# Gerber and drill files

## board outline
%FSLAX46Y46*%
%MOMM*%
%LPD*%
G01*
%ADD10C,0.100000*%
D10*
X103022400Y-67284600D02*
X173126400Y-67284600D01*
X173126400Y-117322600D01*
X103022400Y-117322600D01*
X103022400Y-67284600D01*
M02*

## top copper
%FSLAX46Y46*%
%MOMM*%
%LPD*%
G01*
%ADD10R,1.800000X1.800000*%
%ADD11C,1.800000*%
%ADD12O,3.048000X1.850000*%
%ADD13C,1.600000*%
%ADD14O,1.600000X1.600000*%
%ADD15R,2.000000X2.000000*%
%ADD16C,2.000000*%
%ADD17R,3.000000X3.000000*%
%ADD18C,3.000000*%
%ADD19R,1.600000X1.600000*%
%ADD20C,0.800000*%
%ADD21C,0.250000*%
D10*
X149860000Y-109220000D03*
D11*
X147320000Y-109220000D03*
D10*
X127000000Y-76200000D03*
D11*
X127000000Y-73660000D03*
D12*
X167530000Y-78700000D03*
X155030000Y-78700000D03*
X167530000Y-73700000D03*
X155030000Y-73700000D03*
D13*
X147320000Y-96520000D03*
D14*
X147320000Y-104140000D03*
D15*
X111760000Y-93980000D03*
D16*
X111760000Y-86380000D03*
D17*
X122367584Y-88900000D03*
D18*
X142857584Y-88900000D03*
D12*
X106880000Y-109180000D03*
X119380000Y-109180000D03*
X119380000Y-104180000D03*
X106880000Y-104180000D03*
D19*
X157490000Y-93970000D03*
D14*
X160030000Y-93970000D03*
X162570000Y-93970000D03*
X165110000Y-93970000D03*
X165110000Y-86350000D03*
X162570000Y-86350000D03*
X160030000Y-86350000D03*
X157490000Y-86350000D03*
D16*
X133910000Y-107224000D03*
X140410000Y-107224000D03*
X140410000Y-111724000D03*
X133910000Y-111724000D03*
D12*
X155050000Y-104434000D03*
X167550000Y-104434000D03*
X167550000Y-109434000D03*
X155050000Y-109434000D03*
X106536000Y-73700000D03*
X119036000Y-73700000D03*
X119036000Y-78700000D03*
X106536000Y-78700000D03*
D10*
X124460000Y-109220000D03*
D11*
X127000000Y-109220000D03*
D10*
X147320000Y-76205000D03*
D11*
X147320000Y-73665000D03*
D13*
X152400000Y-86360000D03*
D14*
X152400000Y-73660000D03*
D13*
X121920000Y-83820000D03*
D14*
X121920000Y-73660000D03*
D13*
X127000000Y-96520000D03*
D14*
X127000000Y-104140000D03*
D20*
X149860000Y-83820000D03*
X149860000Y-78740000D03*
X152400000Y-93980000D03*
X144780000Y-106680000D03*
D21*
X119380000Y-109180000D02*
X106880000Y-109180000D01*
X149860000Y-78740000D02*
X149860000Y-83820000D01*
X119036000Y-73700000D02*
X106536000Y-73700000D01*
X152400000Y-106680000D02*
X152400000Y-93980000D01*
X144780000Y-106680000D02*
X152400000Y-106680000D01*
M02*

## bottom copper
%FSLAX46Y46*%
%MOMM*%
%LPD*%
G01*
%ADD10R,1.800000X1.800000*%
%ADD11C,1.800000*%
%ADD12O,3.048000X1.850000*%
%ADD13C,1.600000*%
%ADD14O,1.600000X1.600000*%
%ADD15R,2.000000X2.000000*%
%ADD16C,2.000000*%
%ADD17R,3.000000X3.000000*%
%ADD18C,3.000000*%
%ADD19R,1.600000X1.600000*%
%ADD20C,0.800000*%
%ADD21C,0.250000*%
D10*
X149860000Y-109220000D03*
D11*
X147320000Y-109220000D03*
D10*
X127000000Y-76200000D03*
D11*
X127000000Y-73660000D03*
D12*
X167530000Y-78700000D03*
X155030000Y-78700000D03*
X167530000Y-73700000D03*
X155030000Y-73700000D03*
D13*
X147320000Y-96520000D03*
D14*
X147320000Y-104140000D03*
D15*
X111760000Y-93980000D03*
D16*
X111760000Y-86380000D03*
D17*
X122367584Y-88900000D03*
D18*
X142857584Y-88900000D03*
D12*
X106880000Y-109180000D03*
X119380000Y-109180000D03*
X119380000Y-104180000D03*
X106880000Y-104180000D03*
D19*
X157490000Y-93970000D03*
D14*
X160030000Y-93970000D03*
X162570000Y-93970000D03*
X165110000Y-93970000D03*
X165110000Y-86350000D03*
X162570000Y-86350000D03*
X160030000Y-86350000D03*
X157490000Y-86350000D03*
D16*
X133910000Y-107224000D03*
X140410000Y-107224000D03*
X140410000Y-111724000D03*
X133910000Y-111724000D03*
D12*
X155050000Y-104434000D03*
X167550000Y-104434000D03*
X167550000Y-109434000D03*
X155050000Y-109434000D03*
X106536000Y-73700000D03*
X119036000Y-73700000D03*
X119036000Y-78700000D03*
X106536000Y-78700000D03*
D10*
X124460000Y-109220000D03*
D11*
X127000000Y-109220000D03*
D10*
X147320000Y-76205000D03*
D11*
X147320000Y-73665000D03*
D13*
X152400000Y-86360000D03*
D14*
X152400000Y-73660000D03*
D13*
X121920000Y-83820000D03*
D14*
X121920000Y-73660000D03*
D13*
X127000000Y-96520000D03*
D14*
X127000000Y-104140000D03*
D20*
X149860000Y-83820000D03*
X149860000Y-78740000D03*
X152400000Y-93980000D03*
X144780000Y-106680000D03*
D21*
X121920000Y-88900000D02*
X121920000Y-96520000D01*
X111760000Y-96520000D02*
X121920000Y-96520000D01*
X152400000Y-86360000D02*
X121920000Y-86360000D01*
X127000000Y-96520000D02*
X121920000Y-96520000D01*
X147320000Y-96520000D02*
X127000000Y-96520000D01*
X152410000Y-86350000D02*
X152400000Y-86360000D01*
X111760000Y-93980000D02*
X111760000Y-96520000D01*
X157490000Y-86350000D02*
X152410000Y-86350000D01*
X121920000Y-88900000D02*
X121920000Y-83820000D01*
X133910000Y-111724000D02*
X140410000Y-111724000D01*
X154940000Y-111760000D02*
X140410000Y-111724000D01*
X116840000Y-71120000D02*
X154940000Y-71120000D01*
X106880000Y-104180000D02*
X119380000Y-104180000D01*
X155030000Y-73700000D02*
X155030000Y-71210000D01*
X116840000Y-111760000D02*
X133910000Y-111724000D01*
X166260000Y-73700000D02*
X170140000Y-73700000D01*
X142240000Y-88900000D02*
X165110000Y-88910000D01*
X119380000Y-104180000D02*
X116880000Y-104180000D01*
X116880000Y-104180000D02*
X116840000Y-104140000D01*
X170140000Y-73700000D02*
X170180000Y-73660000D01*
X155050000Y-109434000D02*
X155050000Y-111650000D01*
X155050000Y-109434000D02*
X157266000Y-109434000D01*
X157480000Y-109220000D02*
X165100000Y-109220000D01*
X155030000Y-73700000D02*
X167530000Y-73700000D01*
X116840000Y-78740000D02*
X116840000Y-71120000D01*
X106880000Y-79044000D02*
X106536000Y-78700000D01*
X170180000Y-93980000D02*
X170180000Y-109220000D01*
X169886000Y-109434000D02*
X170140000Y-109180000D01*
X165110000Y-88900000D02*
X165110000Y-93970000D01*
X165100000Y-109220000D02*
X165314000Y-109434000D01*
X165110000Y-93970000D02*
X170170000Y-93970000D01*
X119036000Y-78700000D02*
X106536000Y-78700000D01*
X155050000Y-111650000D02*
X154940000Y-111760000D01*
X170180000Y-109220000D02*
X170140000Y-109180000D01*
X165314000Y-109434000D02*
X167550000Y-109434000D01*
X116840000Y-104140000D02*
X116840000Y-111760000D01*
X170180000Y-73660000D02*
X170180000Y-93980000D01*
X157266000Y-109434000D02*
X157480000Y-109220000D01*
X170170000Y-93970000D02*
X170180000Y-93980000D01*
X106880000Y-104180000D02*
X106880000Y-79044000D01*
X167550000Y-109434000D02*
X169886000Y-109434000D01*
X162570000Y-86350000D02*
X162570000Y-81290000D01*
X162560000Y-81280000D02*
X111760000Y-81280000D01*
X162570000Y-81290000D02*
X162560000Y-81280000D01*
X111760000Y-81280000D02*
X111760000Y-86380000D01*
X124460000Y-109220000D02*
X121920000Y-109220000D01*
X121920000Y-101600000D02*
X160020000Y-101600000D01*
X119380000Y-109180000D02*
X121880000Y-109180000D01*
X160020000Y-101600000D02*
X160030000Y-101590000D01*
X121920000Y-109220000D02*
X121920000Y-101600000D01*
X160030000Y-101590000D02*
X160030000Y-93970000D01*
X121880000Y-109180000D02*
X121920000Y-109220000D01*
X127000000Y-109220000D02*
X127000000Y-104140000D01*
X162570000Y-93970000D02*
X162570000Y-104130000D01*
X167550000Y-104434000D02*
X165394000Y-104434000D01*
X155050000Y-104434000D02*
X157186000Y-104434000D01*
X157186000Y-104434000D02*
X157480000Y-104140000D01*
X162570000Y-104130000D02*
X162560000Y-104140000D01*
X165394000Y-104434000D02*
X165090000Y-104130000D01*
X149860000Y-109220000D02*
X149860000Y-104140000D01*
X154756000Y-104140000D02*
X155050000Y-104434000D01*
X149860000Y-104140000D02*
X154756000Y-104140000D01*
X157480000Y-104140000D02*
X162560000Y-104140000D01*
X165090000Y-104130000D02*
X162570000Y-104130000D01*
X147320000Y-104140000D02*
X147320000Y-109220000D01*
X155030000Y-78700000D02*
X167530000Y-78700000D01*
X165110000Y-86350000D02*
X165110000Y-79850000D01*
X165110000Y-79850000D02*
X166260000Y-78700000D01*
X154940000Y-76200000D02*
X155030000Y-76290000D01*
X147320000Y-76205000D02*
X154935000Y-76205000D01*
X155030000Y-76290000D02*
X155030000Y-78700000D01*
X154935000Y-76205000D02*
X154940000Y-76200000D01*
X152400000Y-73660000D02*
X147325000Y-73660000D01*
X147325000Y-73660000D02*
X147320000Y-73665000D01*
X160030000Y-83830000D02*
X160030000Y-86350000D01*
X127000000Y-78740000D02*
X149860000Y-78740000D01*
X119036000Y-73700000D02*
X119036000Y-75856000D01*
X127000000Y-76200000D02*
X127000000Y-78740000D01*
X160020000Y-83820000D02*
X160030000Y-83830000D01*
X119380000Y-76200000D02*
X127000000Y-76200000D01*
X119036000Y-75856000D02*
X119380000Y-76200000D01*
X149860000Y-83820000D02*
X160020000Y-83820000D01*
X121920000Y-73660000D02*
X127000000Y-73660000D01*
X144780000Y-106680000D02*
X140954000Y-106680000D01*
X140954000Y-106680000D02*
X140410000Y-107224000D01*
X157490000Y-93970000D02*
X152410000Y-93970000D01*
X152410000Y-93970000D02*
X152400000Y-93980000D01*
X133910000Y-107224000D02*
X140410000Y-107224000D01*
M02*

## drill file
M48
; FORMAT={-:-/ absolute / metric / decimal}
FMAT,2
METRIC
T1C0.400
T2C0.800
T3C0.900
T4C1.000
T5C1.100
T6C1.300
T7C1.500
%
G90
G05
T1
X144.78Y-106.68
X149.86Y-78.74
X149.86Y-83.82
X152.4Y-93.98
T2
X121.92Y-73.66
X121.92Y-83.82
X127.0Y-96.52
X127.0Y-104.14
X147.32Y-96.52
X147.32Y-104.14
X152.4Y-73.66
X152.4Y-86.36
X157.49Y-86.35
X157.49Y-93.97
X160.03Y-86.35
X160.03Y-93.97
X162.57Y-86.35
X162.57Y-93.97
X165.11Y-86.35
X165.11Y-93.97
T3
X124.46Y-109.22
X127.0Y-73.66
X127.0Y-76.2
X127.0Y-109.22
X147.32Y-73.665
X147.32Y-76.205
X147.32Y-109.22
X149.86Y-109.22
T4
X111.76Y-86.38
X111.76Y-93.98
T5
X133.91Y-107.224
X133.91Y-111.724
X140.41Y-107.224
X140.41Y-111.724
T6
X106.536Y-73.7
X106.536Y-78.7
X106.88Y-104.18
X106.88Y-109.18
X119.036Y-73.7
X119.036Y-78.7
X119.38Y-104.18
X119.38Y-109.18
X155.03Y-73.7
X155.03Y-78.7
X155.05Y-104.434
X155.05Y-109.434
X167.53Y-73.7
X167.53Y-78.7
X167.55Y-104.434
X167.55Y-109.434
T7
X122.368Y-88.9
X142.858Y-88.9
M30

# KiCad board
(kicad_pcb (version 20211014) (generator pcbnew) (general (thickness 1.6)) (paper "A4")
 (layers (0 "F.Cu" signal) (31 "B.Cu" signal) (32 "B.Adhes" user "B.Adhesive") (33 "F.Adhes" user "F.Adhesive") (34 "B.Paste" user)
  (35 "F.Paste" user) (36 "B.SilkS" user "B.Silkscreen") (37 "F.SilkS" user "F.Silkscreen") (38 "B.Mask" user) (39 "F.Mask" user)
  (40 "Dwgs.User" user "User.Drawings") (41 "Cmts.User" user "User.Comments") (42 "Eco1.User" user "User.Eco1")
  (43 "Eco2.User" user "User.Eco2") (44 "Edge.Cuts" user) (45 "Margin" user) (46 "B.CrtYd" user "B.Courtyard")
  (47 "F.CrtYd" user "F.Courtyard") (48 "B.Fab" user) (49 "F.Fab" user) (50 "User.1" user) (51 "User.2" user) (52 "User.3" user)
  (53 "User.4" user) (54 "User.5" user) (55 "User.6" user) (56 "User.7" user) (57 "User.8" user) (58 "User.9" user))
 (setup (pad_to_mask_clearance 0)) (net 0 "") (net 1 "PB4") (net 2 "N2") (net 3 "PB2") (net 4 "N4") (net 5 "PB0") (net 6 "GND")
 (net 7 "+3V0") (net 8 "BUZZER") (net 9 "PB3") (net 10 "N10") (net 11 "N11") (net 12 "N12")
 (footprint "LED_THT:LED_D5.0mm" (layer "F.Cu") (at 149.86 109.22 180)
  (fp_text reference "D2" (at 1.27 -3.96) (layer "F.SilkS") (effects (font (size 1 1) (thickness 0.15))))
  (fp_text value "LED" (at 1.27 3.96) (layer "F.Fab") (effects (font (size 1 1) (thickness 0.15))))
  (pad "1" thru_hole rect (at 0 0 180) (size 1.8 1.8) (drill 0.9) (layers *.Cu *.Mask) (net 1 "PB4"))
  (pad "2" thru_hole circle (at 2.54 0 180) (size 1.8 1.8) (drill 0.9) (layers *.Cu *.Mask) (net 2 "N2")))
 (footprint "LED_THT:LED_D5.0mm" (layer "F.Cu") (at 127 76.2 90)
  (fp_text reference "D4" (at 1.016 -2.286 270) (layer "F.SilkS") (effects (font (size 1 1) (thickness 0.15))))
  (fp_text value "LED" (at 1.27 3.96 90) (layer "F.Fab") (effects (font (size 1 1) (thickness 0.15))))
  (pad "1" thru_hole rect (at 0 0 90) (size 1.8 1.8) (drill 0.9) (layers *.Cu *.Mask) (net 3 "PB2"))
  (pad "2" thru_hole circle (at 2.54 0 90) (size 1.8 1.8) (drill 0.9) (layers *.Cu *.Mask) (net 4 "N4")))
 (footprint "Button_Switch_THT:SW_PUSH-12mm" (layer "F.Cu") (at 167.53 78.7 180)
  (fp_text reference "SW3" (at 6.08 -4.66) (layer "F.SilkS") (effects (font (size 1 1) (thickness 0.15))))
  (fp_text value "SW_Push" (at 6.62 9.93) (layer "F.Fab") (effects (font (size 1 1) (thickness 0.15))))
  (pad "1" thru_hole oval (at 0 0 180) (size 3.048 1.85) (drill 1.3) (layers *.Cu *.Mask) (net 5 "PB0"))
  (pad "1" thru_hole oval (at 12.5 0 180) (size 3.048 1.85) (drill 1.3) (layers *.Cu *.Mask) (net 5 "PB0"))
  (pad "2" thru_hole oval (at 0 5 180) (size 3.048 1.85) (drill 1.3) (layers *.Cu *.Mask) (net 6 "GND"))
  (pad "2" thru_hole oval (at 12.5 5 180) (size 3.048 1.85) (drill 1.3) (layers *.Cu *.Mask) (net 6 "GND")))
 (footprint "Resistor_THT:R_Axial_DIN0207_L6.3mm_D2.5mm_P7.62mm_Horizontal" (layer "F.Cu") (at 147.32 96.52 -90)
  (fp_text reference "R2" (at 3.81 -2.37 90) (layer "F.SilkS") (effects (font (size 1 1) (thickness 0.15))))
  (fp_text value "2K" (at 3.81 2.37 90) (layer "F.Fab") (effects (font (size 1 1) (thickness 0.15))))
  (pad "1" thru_hole circle (at 0 0 270) (size 1.6 1.6) (drill 0.8) (layers *.Cu *.Mask) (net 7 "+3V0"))
  (pad "2" thru_hole oval (at 7.62 0 270) (size 1.6 1.6) (drill 0.8) (layers *.Cu *.Mask) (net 2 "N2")))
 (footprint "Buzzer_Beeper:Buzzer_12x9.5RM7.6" (layer "F.Cu") (at 111.76 93.98 90)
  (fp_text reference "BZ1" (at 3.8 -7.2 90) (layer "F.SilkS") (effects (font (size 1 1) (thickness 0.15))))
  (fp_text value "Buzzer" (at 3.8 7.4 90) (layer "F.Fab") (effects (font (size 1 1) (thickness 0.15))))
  (pad "1" thru_hole rect (at 0 0 90) (size 2 2) (drill 1) (layers *.Cu *.Mask) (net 7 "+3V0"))
  (pad "2" thru_hole circle (at 7.6 0 90) (size 2 2) (drill 1) (layers *.Cu *.Mask) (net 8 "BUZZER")))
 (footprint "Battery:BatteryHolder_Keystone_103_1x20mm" (layer "F.Cu") (at 122.367584 88.9)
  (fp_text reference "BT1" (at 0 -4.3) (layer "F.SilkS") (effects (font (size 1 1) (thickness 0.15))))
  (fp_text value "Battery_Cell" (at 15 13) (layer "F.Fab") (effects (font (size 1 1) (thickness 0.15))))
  (pad "1" thru_hole rect (at 0 0) (size 3 3) (drill 1.5) (layers *.Cu *.Mask) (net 7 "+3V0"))
  (pad "2" thru_hole circle (at 20.49 0) (size 3 3) (drill 1.5) (layers *.Cu *.Mask) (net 6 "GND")))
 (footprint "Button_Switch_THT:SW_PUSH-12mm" (layer "F.Cu") (at 119.38 109.18 180)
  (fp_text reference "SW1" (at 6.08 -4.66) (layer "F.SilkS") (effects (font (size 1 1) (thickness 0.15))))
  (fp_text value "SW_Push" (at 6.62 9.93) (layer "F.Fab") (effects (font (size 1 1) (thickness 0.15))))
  (pad "1" thru_hole oval (at 12.5 0 180) (size 3.048 1.85) (drill 1.3) (layers *.Cu *.Mask) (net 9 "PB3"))
  (pad "1" thru_hole oval (at 0 0 180) (size 3.048 1.85) (drill 1.3) (layers *.Cu *.Mask) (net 9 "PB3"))
  (pad "2" thru_hole oval (at 0 5 180) (size 3.048 1.85) (drill 1.3) (layers *.Cu *.Mask) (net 6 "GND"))
  (pad "2" thru_hole oval (at 12.5 5 180) (size 3.048 1.85) (drill 1.3) (layers *.Cu *.Mask) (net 6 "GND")))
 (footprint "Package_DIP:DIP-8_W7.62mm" (layer "F.Cu") (at 157.49 93.97 90)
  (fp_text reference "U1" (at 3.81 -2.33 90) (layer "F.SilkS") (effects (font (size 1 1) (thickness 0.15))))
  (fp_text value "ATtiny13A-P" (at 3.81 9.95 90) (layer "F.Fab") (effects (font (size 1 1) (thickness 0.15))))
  (pad "1" thru_hole rect (at 0 0 90) (size 1.6 1.6) (drill 0.8) (layers *.Cu *.Mask) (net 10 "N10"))
  (pad "2" thru_hole oval (at 0 2.54 90) (size 1.6 1.6) (drill 0.8) (layers *.Cu *.Mask) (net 9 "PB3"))
  (pad "3" thru_hole oval (at 0 5.08 90) (size 1.6 1.6) (drill 0.8) (layers *.Cu *.Mask) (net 1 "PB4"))
  (pad "4" thru_hole oval (at 0 7.62 90) (size 1.6 1.6) (drill 0.8) (layers *.Cu *.Mask) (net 6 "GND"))
  (pad "5" thru_hole oval (at 7.62 7.62 90) (size 1.6 1.6) (drill 0.8) (layers *.Cu *.Mask) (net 5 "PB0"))
  (pad "6" thru_hole oval (at 7.62 5.08 90) (size 1.6 1.6) (drill 0.8) (layers *.Cu *.Mask) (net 8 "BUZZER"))
  (pad "7" thru_hole oval (at 7.62 2.54 90) (size 1.6 1.6) (drill 0.8) (layers *.Cu *.Mask) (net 3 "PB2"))
  (pad "8" thru_hole oval (at 7.62 0 90) (size 1.6 1.6) (drill 0.8) (layers *.Cu *.Mask) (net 7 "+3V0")))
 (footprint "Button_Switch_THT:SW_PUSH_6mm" (layer "F.Cu") (at 133.91 107.224)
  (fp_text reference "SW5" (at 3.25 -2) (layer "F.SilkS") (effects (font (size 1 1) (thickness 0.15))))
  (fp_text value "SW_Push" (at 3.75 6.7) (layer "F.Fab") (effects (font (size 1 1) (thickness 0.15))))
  (pad "1" thru_hole circle (at 0 0 90) (size 2 2) (drill 1.1) (layers *.Cu *.Mask) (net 10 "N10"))
  (pad "1" thru_hole circle (at 6.5 0 90) (size 2 2) (drill 1.1) (layers *.Cu *.Mask) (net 10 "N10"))
  (pad "2" thru_hole circle (at 6.5 4.5 90) (size 2 2) (drill 1.1) (layers *.Cu *.Mask) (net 6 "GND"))
  (pad "2" thru_hole circle (at 0 4.5 90) (size 2 2) (drill 1.1) (layers *.Cu *.Mask) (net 6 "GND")))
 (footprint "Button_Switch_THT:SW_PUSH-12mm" (layer "F.Cu") (at 155.05 104.434)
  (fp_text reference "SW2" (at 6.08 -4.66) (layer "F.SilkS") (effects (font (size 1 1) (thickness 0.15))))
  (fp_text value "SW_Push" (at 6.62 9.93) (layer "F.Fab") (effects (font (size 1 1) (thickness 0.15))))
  (pad "1" thru_hole oval (at 0 0) (size 3.048 1.85) (drill 1.3) (layers *.Cu *.Mask) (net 1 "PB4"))
  (pad "1" thru_hole oval (at 12.5 0) (size 3.048 1.85) (drill 1.3) (layers *.Cu *.Mask) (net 1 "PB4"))
  (pad "2" thru_hole oval (at 12.5 5) (size 3.048 1.85) (drill 1.3) (layers *.Cu *.Mask) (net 6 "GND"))
  (pad "2" thru_hole oval (at 0 5) (size 3.048 1.85) (drill 1.3) (layers *.Cu *.Mask) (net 6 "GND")))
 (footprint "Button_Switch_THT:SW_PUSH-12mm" (layer "F.Cu") (at 106.536 73.7)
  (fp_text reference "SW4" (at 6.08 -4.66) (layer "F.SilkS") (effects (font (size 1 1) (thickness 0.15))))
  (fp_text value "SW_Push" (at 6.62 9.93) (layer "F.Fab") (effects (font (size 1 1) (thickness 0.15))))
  (pad "1" thru_hole oval (at 0 0) (size 3.048 1.85) (drill 1.3) (layers *.Cu *.Mask) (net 3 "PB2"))
  (pad "1" thru_hole oval (at 12.5 0) (size 3.048 1.85) (drill 1.3) (layers *.Cu *.Mask) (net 3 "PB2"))
  (pad "2" thru_hole oval (at 12.5 5) (size 3.048 1.85) (drill 1.3) (layers *.Cu *.Mask) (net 6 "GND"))
  (pad "2" thru_hole oval (at 0 5) (size 3.048 1.85) (drill 1.3) (layers *.Cu *.Mask) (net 6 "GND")))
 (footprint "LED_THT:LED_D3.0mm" (layer "F.Cu") (at 124.46 109.22)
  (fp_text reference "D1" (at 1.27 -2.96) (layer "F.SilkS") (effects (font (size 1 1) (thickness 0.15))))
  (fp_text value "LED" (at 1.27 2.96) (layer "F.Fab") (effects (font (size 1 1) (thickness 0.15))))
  (pad "1" thru_hole rect (at 0 0) (size 1.8 1.8) (drill 0.9) (layers *.Cu *.Mask) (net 9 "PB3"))
  (pad "2" thru_hole circle (at 2.54 0) (size 1.8 1.8) (drill 0.9) (layers *.Cu *.Mask) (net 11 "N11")))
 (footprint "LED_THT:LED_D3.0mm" (layer "F.Cu") (at 147.32 76.205 90)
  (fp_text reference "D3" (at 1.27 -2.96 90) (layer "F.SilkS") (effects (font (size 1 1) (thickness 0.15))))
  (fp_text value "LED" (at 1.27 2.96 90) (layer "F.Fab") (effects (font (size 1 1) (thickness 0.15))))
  (pad "1" thru_hole rect (at 0 0 90) (size 1.8 1.8) (drill 0.9) (layers *.Cu *.Mask) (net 5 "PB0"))
  (pad "2" thru_hole circle (at 2.54 0 90) (size 1.8 1.8) (drill 0.9) (layers *.Cu *.Mask) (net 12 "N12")))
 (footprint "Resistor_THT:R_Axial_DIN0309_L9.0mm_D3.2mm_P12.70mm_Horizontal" (layer "F.Cu") (at 152.4 86.36 90)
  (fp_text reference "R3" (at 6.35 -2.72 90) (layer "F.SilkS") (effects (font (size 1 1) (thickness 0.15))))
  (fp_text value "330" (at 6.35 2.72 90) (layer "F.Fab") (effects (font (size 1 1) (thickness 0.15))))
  (pad "1" thru_hole circle (at 0 0 90) (size 1.6 1.6) (drill 0.8) (layers *.Cu *.Mask) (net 7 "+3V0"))
  (pad "2" thru_hole oval (at 12.7 0 90) (size 1.6 1.6) (drill 0.8) (layers *.Cu *.Mask) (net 12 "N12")))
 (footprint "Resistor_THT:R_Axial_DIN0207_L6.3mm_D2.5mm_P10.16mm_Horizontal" (layer "F.Cu") (at 121.92 83.82 90)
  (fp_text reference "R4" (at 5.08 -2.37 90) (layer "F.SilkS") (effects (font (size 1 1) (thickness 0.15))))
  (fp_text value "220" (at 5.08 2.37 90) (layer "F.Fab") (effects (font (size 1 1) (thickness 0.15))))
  (pad "1" thru_hole circle (at 0 0 90) (size 1.6 1.6) (drill 0.8) (layers *.Cu *.Mask) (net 7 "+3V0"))
  (pad "2" thru_hole oval (at 10.16 0 90) (size 1.6 1.6) (drill 0.8) (layers *.Cu *.Mask) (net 4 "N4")))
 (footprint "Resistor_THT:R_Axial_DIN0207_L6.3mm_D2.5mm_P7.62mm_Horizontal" (layer "F.Cu") (at 127 96.52 -90)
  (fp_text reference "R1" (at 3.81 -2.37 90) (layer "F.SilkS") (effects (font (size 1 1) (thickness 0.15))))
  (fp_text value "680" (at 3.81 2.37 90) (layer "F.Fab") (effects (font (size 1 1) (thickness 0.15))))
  (pad "1" thru_hole circle (at 0 0 270) (size 1.6 1.6) (drill 0.8) (layers *.Cu *.Mask) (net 7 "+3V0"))
  (pad "2" thru_hole oval (at 7.62 0 270) (size 1.6 1.6) (drill 0.8) (layers *.Cu *.Mask) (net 11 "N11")))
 (gr_rect (start 103.0224 67.2846) (end 173.1264 117.3226) (layer "Edge.Cuts") (width 0.1) (fill none))
 (segment (start 121.92 88.9) (end 121.92 96.52) (width 0.25) (layer "B.Cu") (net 7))
 (segment (start 111.76 96.52) (end 121.92 96.52) (width 0.25) (layer "B.Cu") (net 7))
 (segment (start 152.4 86.36) (end 121.92 86.36) (width 0.25) (layer "B.Cu") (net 7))
 (segment (start 127 96.52) (end 121.92 96.52) (width 0.25) (layer "B.Cu") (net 7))
 (segment (start 147.32 96.52) (end 127 96.52) (width 0.25) (layer "B.Cu") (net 7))
 (segment (start 152.41 86.35) (end 152.4 86.36) (width 0.25) (layer "B.Cu") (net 7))
 (segment (start 111.76 93.98) (end 111.76 96.52) (width 0.25) (layer "B.Cu") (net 7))
 (segment (start 157.49 86.35) (end 152.41 86.35) (width 0.25) (layer "B.Cu") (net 7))
 (segment (start 121.92 88.9) (end 121.92 83.82) (width 0.25) (layer "B.Cu") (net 7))
 (segment (start 133.91 111.724) (end 140.41 111.724) (width 0.25) (layer "B.Cu") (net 6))
 (segment (start 154.94 111.76) (end 140.41 111.724) (width 0.25) (layer "B.Cu") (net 6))
 (segment (start 116.84 71.12) (end 154.94 71.12) (width 0.25) (layer "B.Cu") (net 6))
 (segment (start 106.88 104.18) (end 119.38 104.18) (width 0.25) (layer "B.Cu") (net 6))
 (segment (start 155.03 73.7) (end 155.03 71.21) (width 0.25) (layer "B.Cu") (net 6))
 (segment (start 116.84 111.76) (end 133.91 111.724) (width 0.25) (layer "B.Cu") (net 6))
 (segment (start 166.26 73.7) (end 170.14 73.7) (width 0.25) (layer "B.Cu") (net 6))
 (segment (start 142.24 88.9) (end 165.11 88.91) (width 0.25) (layer "B.Cu") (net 6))
 (segment (start 119.38 104.18) (end 116.88 104.18) (width 0.25) (layer "B.Cu") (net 6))
 (segment (start 116.88 104.18) (end 116.84 104.14) (width 0.25) (layer "B.Cu") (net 6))
 (segment (start 170.14 73.7) (end 170.18 73.66) (width 0.25) (layer "B.Cu") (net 6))
 (segment (start 155.05 109.434) (end 155.05 111.65) (width 0.25) (layer "B.Cu") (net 6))
 (segment (start 155.05 109.434) (end 157.266 109.434) (width 0.25) (layer "B.Cu") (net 6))
 (segment (start 157.48 109.22) (end 165.1 109.22) (width 0.25) (layer "B.Cu") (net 6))
 (segment (start 155.03 73.7) (end 167.53 73.7) (width 0.25) (layer "B.Cu") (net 6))
 (segment (start 116.84 78.74) (end 116.84 71.12) (width 0.25) (layer "B.Cu") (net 6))
 (segment (start 106.88 79.044) (end 106.536 78.7) (width 0.25) (layer "B.Cu") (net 6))
 (segment (start 170.18 93.98) (end 170.18 109.22) (width 0.25) (layer "B.Cu") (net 6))
 (segment (start 169.886 109.434) (end 170.14 109.18) (width 0.25) (layer "B.Cu") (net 6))
 (segment (start 165.11 88.9) (end 165.11 93.97) (width 0.25) (layer "B.Cu") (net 6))
 (segment (start 165.1 109.22) (end 165.314 109.434) (width 0.25) (layer "B.Cu") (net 6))
 (segment (start 165.11 93.97) (end 170.17 93.97) (width 0.25) (layer "B.Cu") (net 6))
 (segment (start 119.036 78.7) (end 106.536 78.7) (width 0.25) (layer "B.Cu") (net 6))
 (segment (start 155.05 111.65) (end 154.94 111.76) (width 0.25) (layer "B.Cu") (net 6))
 (segment (start 170.18 109.22) (end 170.14 109.18) (width 0.25) (layer "B.Cu") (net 6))
 (segment (start 165.314 109.434) (end 167.55 109.434) (width 0.25) (layer "B.Cu") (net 6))
 (segment (start 116.84 104.14) (end 116.84 111.76) (width 0.25) (layer "B.Cu") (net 6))
 (segment (start 170.18 73.66) (end 170.18 93.98) (width 0.25) (layer "B.Cu") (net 6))
 (segment (start 157.266 109.434) (end 157.48 109.22) (width 0.25) (layer "B.Cu") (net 6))
 (segment (start 170.17 93.97) (end 170.18 93.98) (width 0.25) (layer "B.Cu") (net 6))
 (segment (start 106.88 104.18) (end 106.88 79.044) (width 0.25) (layer "B.Cu") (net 6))
 (segment (start 167.55 109.434) (end 169.886 109.434) (width 0.25) (layer "B.Cu") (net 6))
 (segment (start 162.57 86.35) (end 162.57 81.29) (width 0.25) (layer "B.Cu") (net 8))
 (segment (start 162.56 81.28) (end 111.76 81.28) (width 0.25) (layer "B.Cu") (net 8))
 (segment (start 162.57 81.29) (end 162.56 81.28) (width 0.25) (layer "B.Cu") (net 8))
 (segment (start 111.76 81.28) (end 111.76 86.38) (width 0.25) (layer "B.Cu") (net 8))
 (segment (start 119.38 109.18) (end 106.88 109.18) (width 0.25) (layer "F.Cu") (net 9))
 (segment (start 124.46 109.22) (end 121.92 109.22) (width 0.25) (layer "B.Cu") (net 9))
 (segment (start 121.92 101.6) (end 160.02 101.6) (width 0.25) (layer "B.Cu") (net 9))
 (segment (start 119.38 109.18) (end 121.88 109.18) (width 0.25) (layer "B.Cu") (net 9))
 (segment (start 160.02 101.6) (end 160.03 101.59) (width 0.25) (layer "B.Cu") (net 9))
 (segment (start 121.92 109.22) (end 121.92 101.6) (width 0.25) (layer "B.Cu") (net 9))
 (segment (start 160.03 101.59) (end 160.03 93.97) (width 0.25) (layer "B.Cu") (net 9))
 (segment (start 121.88 109.18) (end 121.92 109.22) (width 0.25) (layer "B.Cu") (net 9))
 (segment (start 127 109.22) (end 127 104.14) (width 0.25) (layer "B.Cu") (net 11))
 (segment (start 162.57 93.97) (end 162.57 104.13) (width 0.25) (layer "B.Cu") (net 1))
 (segment (start 167.55 104.434) (end 165.394 104.434) (width 0.25) (layer "B.Cu") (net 1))
 (segment (start 155.05 104.434) (end 157.186 104.434) (width 0.25) (layer "B.Cu") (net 1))
 (segment (start 157.186 104.434) (end 157.48 104.14) (width 0.25) (layer "B.Cu") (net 1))
 (segment (start 162.57 104.13) (end 162.56 104.14) (width 0.25) (layer "B.Cu") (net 1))
 (segment (start 165.394 104.434) (end 165.09 104.13) (width 0.25) (layer "B.Cu") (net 1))
 (segment (start 149.86 109.22) (end 149.86 104.14) (width 0.25) (layer "B.Cu") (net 1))
 (segment (start 154.756 104.14) (end 155.05 104.434) (width 0.25) (layer "B.Cu") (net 1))
 (segment (start 149.86 104.14) (end 154.756 104.14) (width 0.25) (layer "B.Cu") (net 1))
 (segment (start 157.48 104.14) (end 162.56 104.14) (width 0.25) (layer "B.Cu") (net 1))
 (segment (start 165.09 104.13) (end 162.57 104.13) (width 0.25) (layer "B.Cu") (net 1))
 (segment (start 147.32 104.14) (end 147.32 109.22) (width 0.25) (layer "B.Cu") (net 2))
 (segment (start 155.03 78.7) (end 167.53 78.7) (width 0.25) (layer "B.Cu") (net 5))
 (segment (start 165.11 86.35) (end 165.11 79.85) (width 0.25) (layer "B.Cu") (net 5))
 (segment (start 165.11 79.85) (end 166.26 78.7) (width 0.25) (layer "B.Cu") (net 5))
 (segment (start 154.94 76.2) (end 155.03 76.29) (width 0.25) (layer "B.Cu") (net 5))
 (segment (start 147.32 76.205) (end 154.935 76.205) (width 0.25) (layer "B.Cu") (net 5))
 (segment (start 155.03 76.29) (end 155.03 78.7) (width 0.25) (layer "B.Cu") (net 5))
 (segment (start 154.935 76.205) (end 154.94 76.2) (width 0.25) (layer "B.Cu") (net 5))
 (segment (start 152.4 73.66) (end 147.325 73.66) (width 0.25) (layer "B.Cu") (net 12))
 (segment (start 147.325 73.66) (end 147.32 73.665) (width 0.25) (layer "B.Cu") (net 12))
 (segment (start 149.86 78.74) (end 149.86 83.82) (width 0.25) (layer "F.Cu") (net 3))
 (segment (start 119.036 73.7) (end 106.536 73.7) (width 0.25) (layer "F.Cu") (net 3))
 (via (at 149.86 83.82) (size 0.8) (drill 0.4) (layers "F.Cu" "B.Cu") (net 3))
 (via (at 149.86 78.74) (size 0.8) (drill 0.4) (layers "F.Cu" "B.Cu") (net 3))
 (segment (start 160.03 83.83) (end 160.03 86.35) (width 0.25) (layer "B.Cu") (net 3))
 (segment (start 127 78.74) (end 149.86 78.74) (width 0.25) (layer "B.Cu") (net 3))
 (segment (start 119.036 73.7) (end 119.036 75.856) (width 0.25) (layer "B.Cu") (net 3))
 (segment (start 127 76.2) (end 127 78.74) (width 0.25) (layer "B.Cu") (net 3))
 (segment (start 160.02 83.82) (end 160.03 83.83) (width 0.25) (layer "B.Cu") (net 3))
 (segment (start 119.38 76.2) (end 127 76.2) (width 0.25) (layer "B.Cu") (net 3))
 (segment (start 119.036 75.856) (end 119.38 76.2) (width 0.25) (layer "B.Cu") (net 3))
 (segment (start 149.86 83.82) (end 160.02 83.82) (width 0.25) (layer "B.Cu") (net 3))
 (segment (start 121.92 73.66) (end 127 73.66) (width 0.25) (layer "B.Cu") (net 4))
 (segment (start 152.4 106.68) (end 152.4 93.98) (width 0.25) (layer "F.Cu") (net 10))
 (segment (start 144.78 106.68) (end 152.4 106.68) (width 0.25) (layer "F.Cu") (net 10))
 (via (at 152.4 93.98) (size 0.8) (drill 0.4) (layers "F.Cu" "B.Cu") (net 10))
 (via (at 144.78 106.68) (size 0.8) (drill 0.4) (layers "F.Cu" "B.Cu") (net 10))
 (segment (start 144.78 106.68) (end 140.954 106.68) (width 0.25) (layer "B.Cu") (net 10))
 (segment (start 140.954 106.68) (end 140.41 107.224) (width 0.25) (layer "B.Cu") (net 10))
 (segment (start 157.49 93.97) (end 152.41 93.97) (width 0.25) (layer "B.Cu") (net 10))
 (segment (start 152.41 93.97) (end 152.4 93.98) (width 0.25) (layer "B.Cu") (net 10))
 (segment (start 133.91 107.224) (end 140.41 107.224) (width 0.25) (layer "B.Cu") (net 10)))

